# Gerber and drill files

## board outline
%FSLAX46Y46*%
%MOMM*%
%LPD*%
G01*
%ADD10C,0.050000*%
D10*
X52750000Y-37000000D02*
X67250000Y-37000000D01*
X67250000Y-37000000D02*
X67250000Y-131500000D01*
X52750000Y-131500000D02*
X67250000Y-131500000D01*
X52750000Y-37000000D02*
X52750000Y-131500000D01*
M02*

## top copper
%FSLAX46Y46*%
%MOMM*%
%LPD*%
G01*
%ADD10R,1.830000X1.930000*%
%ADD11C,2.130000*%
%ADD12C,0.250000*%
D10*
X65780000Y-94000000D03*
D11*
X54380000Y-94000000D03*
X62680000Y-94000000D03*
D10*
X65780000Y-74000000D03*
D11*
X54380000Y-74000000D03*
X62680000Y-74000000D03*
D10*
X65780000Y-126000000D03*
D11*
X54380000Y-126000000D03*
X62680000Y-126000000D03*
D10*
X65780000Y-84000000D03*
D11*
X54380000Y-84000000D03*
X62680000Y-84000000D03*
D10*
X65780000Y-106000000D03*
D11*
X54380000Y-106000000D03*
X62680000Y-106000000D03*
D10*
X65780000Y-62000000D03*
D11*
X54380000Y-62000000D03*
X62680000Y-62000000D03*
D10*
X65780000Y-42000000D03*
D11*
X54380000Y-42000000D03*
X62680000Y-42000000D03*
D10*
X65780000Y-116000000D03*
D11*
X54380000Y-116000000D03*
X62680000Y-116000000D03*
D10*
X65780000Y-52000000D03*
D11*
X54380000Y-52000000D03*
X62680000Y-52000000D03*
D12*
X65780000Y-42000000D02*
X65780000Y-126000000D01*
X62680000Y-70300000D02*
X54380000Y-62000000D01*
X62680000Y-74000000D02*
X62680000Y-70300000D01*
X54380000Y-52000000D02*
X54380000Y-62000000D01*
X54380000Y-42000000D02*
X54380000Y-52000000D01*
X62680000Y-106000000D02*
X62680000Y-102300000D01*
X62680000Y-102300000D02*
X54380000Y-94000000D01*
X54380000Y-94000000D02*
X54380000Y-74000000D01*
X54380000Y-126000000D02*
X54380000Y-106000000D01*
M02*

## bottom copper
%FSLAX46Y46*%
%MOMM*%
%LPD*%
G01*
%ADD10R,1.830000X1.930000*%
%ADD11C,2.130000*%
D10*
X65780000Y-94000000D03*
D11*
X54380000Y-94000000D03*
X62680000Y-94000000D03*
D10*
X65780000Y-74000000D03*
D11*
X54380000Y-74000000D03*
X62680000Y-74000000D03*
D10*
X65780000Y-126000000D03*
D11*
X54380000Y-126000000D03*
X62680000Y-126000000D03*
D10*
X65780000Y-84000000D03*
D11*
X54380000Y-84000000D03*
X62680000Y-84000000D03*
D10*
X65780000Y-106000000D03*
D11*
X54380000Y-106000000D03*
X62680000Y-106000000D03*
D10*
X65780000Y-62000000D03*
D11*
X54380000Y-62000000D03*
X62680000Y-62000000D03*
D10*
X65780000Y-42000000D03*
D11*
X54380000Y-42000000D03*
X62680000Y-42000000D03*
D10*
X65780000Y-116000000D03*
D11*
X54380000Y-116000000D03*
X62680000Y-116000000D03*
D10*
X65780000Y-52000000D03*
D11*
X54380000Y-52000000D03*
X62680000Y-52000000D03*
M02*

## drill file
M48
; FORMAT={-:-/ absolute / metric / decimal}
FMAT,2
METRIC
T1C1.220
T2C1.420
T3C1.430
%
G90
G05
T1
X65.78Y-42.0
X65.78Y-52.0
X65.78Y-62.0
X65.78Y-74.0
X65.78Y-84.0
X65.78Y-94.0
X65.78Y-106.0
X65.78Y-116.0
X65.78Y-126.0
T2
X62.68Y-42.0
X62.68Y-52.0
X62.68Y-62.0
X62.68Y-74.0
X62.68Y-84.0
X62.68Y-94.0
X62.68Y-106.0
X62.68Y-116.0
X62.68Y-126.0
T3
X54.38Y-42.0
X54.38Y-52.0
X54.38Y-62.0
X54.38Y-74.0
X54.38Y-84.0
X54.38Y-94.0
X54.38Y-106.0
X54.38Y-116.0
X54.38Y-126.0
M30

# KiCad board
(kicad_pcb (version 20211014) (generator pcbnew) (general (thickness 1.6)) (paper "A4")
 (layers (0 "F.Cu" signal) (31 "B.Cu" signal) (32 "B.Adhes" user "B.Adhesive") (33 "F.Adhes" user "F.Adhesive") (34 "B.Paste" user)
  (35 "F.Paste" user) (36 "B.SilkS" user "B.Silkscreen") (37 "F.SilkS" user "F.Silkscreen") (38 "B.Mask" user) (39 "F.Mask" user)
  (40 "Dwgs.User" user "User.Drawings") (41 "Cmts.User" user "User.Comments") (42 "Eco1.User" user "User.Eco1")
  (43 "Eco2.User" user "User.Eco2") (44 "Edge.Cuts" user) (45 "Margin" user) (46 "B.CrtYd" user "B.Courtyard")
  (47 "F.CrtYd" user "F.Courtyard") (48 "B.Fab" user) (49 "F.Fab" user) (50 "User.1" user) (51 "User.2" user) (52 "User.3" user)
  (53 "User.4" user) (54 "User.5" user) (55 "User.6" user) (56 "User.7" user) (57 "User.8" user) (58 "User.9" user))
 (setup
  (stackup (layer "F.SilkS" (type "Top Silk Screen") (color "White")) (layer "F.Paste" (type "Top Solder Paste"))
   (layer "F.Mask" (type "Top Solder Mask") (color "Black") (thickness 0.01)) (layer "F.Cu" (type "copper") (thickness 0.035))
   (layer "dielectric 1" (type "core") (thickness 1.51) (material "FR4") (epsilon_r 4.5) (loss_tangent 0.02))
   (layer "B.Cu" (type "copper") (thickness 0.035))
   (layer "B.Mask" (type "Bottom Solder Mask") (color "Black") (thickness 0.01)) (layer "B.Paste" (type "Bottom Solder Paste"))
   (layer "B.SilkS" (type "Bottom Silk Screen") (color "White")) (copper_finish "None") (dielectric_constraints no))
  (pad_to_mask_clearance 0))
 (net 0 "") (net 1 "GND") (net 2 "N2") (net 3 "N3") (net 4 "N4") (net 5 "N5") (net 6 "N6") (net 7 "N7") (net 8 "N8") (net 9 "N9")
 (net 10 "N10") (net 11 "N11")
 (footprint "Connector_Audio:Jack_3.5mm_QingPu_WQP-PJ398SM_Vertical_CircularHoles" (layer "F.Cu") (at 65.78 94 -90)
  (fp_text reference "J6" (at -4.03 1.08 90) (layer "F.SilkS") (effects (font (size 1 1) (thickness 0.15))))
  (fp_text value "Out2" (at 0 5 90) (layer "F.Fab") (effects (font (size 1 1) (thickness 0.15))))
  (pad "S" thru_hole rect locked (at 0 0 90) (size 1.93 1.83) (drill 1.22) (layers *.Cu *.Mask) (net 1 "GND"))
  (pad "T" thru_hole circle locked (at 0 11.4 90) (size 2.13 2.13) (drill 1.43) (layers *.Cu *.Mask) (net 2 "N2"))
  (pad "TN" thru_hole circle locked (at 0 3.1 90) (size 2.13 2.13) (drill 1.42) (layers *.Cu *.Mask) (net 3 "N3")))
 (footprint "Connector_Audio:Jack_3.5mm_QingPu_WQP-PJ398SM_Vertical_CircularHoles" (layer "F.Cu") (at 65.78 74 -90)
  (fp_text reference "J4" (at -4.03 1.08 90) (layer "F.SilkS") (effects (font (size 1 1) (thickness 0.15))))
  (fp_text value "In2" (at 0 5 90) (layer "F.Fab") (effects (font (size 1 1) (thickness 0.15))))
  (pad "S" thru_hole rect locked (at 0 0 90) (size 1.93 1.83) (drill 1.22) (layers *.Cu *.Mask) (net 1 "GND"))
  (pad "T" thru_hole circle locked (at 0 11.4 90) (size 2.13 2.13) (drill 1.43) (layers *.Cu *.Mask) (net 2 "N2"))
  (pad "TN" thru_hole circle locked (at 0 3.1 90) (size 2.13 2.13) (drill 1.42) (layers *.Cu *.Mask) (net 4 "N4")))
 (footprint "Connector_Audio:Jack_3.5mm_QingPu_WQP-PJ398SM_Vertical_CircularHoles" (layer "F.Cu") (at 65.78 126 -90)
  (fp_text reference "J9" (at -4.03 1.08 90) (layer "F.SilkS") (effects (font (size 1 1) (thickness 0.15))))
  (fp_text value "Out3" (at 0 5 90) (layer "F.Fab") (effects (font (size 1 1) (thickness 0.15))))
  (pad "S" thru_hole rect locked (at 0 0 90) (size 1.93 1.83) (drill 1.22) (layers *.Cu *.Mask) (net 1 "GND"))
  (pad "T" thru_hole circle locked (at 0 11.4 90) (size 2.13 2.13) (drill 1.43) (layers *.Cu *.Mask) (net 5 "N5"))
  (pad "TN" thru_hole circle locked (at 0 3.1 90) (size 2.13 2.13) (drill 1.42) (layers *.Cu *.Mask) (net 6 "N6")))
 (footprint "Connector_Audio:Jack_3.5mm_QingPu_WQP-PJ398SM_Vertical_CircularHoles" (layer "F.Cu") (at 65.78 84 -90)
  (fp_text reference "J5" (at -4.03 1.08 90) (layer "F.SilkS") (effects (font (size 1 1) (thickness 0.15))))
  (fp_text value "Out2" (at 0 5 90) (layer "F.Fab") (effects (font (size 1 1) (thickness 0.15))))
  (pad "S" thru_hole rect locked (at 0 0 90) (size 1.93 1.83) (drill 1.22) (layers *.Cu *.Mask) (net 1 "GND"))
  (pad "T" thru_hole circle locked (at 0 11.4 90) (size 2.13 2.13) (drill 1.43) (layers *.Cu *.Mask) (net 2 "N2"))
  (pad "TN" thru_hole circle locked (at 0 3.1 90) (size 2.13 2.13) (drill 1.42) (layers *.Cu *.Mask) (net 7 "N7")))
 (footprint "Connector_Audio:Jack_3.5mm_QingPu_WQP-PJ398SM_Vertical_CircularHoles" (layer "F.Cu") (at 65.78 106 -90)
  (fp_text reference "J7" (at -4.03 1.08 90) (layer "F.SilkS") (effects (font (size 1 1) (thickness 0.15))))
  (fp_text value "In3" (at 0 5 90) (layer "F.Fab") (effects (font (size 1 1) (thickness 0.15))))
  (pad "S" thru_hole rect locked (at 0 0 90) (size 1.93 1.83) (drill 1.22) (layers *.Cu *.Mask) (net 1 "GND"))
  (pad "T" thru_hole circle locked (at 0 11.4 90) (size 2.13 2.13) (drill 1.43) (layers *.Cu *.Mask) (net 5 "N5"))
  (pad "TN" thru_hole circle locked (at 0 3.1 90) (size 2.13 2.13) (drill 1.42) (layers *.Cu *.Mask) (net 2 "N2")))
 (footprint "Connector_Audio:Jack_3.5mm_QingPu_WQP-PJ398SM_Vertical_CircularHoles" (layer "F.Cu") (at 65.78 62 -90)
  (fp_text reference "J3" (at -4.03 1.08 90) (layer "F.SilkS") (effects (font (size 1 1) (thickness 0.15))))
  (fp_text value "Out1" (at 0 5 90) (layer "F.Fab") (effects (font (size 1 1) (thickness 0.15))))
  (pad "S" thru_hole rect locked (at 0 0 90) (size 1.93 1.83) (drill 1.22) (layers *.Cu *.Mask) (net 1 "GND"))
  (pad "T" thru_hole circle locked (at 0 11.4 90) (size 2.13 2.13) (drill 1.43) (layers *.Cu *.Mask) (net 4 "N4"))
  (pad "TN" thru_hole circle locked (at 0 3.1 90) (size 2.13 2.13) (drill 1.42) (layers *.Cu *.Mask) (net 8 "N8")))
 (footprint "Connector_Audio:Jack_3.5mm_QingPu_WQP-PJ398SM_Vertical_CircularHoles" (layer "F.Cu") (at 65.78 42 -90)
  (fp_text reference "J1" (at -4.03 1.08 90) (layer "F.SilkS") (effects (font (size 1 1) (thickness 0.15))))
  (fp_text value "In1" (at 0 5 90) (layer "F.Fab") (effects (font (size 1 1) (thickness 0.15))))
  (pad "S" thru_hole rect locked (at 0 0 90) (size 1.93 1.83) (drill 1.22) (layers *.Cu *.Mask) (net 1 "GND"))
  (pad "T" thru_hole circle locked (at 0 11.4 90) (size 2.13 2.13) (drill 1.43) (layers *.Cu *.Mask) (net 4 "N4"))
  (pad "TN" thru_hole circle locked (at 0 3.1 90) (size 2.13 2.13) (drill 1.42) (layers *.Cu *.Mask) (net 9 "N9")))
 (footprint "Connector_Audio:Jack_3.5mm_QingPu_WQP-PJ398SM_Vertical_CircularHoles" (layer "F.Cu") (at 65.78 116 -90)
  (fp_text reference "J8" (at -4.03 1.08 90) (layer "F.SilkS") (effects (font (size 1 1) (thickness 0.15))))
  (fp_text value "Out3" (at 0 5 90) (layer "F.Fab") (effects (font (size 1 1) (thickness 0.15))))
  (pad "S" thru_hole rect locked (at 0 0 90) (size 1.93 1.83) (drill 1.22) (layers *.Cu *.Mask) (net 1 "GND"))
  (pad "T" thru_hole circle locked (at 0 11.4 90) (size 2.13 2.13) (drill 1.43) (layers *.Cu *.Mask) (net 5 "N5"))
  (pad "TN" thru_hole circle locked (at 0 3.1 90) (size 2.13 2.13) (drill 1.42) (layers *.Cu *.Mask) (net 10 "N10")))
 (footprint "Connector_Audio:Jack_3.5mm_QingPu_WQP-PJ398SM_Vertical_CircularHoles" (layer "F.Cu") (at 65.78 52 -90)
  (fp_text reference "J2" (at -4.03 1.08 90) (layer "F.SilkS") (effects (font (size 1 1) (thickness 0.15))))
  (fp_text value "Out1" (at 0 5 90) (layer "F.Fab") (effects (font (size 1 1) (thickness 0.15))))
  (pad "S" thru_hole rect locked (at 0 0 90) (size 1.93 1.83) (drill 1.22) (layers *.Cu *.Mask) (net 1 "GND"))
  (pad "T" thru_hole circle locked (at 0 11.4 90) (size 2.13 2.13) (drill 1.43) (layers *.Cu *.Mask) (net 4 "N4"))
  (pad "TN" thru_hole circle locked (at 0 3.1 90) (size 2.13 2.13) (drill 1.42) (layers *.Cu *.Mask) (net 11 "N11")))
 (gr_line (start 52.75 37) (end 67.25 37) (layer "Edge.Cuts") (width 0.05))
 (gr_line (start 67.25 37) (end 67.25 131.5) (layer "Edge.Cuts") (width 0.05))
 (gr_line (start 52.75 131.5) (end 67.25 131.5) (layer "Edge.Cuts") (width 0.05))
 (gr_line (start 52.75 37) (end 52.75 131.5) (layer "Edge.Cuts") (width 0.05))
 (segment (start 65.78 42) (end 65.78 126) (width 0.25) (layer "F.Cu") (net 1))
 (segment (start 62.68 70.3) (end 54.38 62) (width 0.25) (layer "F.Cu") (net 4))
 (segment (start 62.68 74) (end 62.68 70.3) (width 0.25) (layer "F.Cu") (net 4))
 (segment (start 54.38 52) (end 54.38 62) (width 0.25) (layer "F.Cu") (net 4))
 (segment (start 54.38 42) (end 54.38 52) (width 0.25) (layer "F.Cu") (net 4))
 (segment (start 62.68 106) (end 62.68 102.3) (width 0.25) (layer "F.Cu") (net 2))
 (segment (start 62.68 102.3) (end 54.38 94) (width 0.25) (layer "F.Cu") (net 2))
 (segment (start 54.38 94) (end 54.38 74) (width 0.25) (layer "F.Cu") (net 2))
 (segment (start 54.38 126) (end 54.38 106) (width 0.25) (layer "F.Cu") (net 5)))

